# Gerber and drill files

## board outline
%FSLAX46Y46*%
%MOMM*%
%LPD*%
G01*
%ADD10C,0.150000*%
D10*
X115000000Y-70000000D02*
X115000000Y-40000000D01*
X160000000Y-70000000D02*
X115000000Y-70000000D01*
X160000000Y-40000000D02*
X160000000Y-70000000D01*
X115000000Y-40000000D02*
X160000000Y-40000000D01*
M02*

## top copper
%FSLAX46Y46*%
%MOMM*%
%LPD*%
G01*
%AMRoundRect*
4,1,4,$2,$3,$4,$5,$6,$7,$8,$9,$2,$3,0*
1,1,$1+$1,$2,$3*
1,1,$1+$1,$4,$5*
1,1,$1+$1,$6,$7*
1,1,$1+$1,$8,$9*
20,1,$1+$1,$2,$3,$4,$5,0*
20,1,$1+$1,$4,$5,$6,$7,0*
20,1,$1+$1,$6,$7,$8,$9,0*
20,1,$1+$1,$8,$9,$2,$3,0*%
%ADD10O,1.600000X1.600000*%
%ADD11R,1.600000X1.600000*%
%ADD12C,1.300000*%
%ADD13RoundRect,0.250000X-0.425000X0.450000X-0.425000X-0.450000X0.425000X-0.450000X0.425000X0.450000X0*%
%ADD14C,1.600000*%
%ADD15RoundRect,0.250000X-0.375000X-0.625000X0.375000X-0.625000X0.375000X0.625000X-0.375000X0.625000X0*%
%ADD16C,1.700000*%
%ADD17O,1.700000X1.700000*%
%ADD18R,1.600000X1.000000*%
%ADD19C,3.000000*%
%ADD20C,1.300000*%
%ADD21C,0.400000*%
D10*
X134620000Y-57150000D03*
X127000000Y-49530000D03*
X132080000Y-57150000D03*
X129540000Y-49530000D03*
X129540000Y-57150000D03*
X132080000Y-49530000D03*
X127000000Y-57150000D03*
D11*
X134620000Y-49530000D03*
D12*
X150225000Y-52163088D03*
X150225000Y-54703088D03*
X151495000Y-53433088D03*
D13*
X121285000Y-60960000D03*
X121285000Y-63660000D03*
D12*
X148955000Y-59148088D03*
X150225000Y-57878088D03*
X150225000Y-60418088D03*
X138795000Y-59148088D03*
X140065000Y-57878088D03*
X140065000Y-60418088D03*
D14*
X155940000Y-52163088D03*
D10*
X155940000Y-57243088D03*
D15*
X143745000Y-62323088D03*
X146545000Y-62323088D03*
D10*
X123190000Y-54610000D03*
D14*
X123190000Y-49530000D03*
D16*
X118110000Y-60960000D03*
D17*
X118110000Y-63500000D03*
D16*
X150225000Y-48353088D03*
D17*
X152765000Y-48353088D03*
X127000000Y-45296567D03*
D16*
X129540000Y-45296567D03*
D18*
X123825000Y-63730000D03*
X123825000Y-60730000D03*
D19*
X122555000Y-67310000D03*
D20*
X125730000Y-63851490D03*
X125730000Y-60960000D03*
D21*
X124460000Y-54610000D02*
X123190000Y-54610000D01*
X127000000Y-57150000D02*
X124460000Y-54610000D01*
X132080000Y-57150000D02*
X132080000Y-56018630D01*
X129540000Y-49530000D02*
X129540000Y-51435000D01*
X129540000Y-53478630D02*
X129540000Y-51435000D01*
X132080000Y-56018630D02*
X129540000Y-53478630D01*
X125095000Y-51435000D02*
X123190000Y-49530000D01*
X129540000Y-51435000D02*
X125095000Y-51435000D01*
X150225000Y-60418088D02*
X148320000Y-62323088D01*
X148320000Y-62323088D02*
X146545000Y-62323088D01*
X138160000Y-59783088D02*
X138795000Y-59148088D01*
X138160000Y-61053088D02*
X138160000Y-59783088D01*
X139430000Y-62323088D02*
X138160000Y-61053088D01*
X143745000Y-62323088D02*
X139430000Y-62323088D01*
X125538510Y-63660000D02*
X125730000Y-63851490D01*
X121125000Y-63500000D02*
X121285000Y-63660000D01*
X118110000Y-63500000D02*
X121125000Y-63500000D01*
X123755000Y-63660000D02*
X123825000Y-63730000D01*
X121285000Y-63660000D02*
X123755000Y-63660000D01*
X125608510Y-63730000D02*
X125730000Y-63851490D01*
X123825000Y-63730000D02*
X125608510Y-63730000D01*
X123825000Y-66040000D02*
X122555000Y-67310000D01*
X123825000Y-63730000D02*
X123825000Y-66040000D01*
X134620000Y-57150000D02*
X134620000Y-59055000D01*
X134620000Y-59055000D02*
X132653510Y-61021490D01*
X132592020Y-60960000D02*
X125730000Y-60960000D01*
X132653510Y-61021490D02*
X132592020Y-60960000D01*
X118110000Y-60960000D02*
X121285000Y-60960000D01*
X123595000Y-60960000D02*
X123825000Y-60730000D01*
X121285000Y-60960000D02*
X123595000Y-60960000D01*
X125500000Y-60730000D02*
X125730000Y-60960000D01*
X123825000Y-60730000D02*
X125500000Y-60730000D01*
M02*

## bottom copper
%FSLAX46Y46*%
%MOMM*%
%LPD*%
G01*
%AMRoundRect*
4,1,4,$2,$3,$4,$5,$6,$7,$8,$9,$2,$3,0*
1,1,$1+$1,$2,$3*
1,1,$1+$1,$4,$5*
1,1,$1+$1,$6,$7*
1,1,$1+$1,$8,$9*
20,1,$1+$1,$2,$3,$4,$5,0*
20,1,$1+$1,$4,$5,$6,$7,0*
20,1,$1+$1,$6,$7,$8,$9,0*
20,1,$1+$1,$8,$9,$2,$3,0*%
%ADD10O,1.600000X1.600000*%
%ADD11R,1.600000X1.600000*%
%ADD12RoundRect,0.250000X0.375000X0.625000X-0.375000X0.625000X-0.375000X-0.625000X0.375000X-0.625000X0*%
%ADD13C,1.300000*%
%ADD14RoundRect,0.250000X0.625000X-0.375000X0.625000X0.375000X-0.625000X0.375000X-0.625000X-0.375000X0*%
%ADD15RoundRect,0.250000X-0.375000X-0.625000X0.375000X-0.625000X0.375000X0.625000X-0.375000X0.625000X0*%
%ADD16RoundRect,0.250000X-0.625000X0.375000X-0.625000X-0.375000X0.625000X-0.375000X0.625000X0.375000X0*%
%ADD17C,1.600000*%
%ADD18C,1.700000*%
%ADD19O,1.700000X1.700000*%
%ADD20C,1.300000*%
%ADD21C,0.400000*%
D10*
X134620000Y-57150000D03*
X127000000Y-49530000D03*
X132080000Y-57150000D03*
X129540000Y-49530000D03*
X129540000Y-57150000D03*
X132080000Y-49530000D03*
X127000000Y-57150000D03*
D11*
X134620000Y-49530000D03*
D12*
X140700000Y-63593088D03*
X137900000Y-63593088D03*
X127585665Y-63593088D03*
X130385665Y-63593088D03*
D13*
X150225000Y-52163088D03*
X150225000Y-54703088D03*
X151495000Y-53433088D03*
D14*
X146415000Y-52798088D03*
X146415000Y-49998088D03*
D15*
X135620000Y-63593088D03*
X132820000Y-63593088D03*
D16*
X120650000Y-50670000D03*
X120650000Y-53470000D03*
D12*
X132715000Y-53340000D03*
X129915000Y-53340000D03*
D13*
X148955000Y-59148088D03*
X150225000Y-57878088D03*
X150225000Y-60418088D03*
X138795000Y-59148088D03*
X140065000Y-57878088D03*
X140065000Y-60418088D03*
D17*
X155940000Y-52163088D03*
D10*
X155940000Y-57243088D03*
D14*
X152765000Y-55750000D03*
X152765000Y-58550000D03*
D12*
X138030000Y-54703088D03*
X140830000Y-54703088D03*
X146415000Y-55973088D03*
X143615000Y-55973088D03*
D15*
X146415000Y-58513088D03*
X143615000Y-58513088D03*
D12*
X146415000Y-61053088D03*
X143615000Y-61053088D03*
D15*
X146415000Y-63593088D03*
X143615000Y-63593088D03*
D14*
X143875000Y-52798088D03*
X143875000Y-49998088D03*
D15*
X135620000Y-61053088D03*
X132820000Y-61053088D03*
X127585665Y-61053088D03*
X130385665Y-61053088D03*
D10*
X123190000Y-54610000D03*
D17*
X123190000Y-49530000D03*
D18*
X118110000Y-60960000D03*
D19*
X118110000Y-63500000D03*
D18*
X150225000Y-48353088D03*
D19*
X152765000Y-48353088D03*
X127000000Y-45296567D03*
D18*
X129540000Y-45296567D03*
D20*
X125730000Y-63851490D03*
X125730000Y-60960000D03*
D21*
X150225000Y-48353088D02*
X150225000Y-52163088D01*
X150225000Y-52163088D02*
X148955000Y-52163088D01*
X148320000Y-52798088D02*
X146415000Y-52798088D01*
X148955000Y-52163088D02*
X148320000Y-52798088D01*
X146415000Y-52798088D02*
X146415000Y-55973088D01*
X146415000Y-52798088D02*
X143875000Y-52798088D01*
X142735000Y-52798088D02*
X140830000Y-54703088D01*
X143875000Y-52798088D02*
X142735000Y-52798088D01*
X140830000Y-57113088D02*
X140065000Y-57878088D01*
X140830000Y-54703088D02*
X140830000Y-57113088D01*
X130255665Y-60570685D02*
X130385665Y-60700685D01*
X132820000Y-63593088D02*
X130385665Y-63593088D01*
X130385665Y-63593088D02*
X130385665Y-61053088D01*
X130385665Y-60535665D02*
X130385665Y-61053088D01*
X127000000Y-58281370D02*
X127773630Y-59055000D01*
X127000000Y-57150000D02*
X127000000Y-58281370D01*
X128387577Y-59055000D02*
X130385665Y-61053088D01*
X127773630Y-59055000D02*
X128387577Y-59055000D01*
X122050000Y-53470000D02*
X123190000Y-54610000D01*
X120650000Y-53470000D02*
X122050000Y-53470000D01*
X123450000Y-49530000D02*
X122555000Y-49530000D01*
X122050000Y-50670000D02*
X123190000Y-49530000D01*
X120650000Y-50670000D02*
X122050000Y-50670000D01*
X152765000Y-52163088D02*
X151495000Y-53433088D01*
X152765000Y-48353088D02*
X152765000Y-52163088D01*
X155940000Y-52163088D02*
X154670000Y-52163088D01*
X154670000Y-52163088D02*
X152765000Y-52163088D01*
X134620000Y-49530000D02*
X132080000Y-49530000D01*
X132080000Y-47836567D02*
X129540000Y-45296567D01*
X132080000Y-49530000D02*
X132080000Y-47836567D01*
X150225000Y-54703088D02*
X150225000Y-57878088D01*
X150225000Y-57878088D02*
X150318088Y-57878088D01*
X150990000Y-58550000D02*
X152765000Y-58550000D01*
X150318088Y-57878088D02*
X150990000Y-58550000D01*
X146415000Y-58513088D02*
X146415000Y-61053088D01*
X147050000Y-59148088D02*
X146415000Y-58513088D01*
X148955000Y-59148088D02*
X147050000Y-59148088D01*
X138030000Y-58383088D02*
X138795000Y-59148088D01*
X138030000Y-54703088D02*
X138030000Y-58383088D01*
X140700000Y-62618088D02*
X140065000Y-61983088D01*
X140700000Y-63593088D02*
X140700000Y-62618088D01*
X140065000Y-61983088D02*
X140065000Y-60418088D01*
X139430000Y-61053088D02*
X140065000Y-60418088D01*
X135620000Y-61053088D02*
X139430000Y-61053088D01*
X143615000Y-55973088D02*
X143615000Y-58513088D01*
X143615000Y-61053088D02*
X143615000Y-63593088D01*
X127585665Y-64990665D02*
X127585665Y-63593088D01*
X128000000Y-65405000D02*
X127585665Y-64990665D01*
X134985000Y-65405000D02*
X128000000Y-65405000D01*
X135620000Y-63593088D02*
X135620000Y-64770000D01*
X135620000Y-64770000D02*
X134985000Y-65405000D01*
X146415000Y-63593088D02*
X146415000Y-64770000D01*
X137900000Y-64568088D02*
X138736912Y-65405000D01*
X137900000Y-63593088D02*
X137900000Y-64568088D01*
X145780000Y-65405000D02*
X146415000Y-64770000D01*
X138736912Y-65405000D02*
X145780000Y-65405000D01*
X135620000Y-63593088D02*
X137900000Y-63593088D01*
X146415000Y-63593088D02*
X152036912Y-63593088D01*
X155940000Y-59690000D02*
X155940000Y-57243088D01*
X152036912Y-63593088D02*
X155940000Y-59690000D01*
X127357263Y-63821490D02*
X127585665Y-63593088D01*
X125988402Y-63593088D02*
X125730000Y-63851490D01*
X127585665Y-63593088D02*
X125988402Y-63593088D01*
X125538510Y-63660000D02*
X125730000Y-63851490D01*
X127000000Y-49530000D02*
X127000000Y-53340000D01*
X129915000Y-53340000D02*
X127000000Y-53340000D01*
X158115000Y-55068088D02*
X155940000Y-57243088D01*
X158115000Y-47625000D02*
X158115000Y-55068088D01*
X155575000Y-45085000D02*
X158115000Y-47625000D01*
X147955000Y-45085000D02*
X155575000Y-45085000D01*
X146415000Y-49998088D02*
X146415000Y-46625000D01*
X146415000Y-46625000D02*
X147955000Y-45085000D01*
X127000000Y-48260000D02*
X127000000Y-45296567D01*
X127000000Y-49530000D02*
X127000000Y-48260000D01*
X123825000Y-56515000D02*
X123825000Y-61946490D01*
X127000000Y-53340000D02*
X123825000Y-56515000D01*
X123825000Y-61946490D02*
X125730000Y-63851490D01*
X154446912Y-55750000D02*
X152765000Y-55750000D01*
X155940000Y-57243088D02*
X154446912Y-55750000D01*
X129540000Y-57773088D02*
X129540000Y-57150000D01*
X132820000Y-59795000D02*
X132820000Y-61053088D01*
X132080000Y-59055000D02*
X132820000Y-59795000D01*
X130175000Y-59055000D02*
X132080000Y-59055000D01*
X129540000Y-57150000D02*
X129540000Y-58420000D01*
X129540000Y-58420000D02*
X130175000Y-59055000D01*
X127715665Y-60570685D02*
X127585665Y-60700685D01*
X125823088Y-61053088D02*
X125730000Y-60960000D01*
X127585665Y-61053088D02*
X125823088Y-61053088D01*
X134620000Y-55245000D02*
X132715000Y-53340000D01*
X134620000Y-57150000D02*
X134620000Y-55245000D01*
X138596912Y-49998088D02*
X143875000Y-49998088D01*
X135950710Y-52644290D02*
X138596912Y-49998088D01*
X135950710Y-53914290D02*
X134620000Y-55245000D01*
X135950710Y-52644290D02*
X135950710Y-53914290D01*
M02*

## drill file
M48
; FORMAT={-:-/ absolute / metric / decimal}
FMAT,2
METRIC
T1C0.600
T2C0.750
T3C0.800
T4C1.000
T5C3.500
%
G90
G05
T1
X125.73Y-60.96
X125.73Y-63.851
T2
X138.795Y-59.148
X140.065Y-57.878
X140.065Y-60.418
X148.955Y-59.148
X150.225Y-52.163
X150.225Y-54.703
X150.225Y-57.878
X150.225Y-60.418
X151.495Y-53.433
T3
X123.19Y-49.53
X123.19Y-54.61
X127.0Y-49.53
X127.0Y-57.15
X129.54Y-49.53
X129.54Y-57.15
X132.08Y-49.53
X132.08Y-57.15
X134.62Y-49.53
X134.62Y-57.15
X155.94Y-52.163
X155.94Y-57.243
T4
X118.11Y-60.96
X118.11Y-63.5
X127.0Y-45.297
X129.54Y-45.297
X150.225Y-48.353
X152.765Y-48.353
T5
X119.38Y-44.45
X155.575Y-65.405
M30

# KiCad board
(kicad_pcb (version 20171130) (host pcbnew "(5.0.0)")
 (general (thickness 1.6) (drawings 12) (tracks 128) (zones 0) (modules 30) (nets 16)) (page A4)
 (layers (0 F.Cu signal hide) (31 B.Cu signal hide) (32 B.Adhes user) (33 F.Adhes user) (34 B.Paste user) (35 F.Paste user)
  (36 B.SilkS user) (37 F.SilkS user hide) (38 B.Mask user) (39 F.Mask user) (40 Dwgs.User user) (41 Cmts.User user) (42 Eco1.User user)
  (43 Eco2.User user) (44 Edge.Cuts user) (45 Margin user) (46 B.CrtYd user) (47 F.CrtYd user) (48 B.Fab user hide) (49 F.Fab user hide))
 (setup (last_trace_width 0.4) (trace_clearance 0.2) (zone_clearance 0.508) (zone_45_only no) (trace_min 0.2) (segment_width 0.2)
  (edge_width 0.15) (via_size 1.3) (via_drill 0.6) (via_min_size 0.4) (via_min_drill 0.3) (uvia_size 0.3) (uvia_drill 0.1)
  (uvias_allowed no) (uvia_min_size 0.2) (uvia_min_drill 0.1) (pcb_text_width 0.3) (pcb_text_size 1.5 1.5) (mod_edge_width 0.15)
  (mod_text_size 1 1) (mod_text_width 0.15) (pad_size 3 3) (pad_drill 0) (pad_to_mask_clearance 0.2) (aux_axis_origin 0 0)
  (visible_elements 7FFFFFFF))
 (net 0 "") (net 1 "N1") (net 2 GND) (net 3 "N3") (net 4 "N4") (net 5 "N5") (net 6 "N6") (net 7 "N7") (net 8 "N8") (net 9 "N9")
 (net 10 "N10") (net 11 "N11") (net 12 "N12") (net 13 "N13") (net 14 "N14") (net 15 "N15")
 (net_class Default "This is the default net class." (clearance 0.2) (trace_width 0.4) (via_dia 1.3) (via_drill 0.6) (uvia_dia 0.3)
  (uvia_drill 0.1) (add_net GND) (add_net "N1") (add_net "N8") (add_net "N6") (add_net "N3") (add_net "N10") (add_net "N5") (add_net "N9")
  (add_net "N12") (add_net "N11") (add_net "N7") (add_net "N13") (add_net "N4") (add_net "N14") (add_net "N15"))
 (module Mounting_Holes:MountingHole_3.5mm (layer F.Cu) (at 119.38 44.45)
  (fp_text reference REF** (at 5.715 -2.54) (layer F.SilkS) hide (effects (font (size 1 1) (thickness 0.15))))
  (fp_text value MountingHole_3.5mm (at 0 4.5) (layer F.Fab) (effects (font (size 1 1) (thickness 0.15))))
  (pad 1 np_thru_hole circle (at 0 0) (size 3.5 3.5) (drill 3.5) (layers *.Cu *.Mask)))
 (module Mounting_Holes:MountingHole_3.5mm (layer F.Cu) (at 155.575 65.405)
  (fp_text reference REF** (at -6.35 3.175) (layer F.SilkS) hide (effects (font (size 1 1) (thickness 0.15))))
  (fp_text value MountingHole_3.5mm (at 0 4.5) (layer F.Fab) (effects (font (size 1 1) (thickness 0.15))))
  (pad 1 np_thru_hole circle (at 0 0) (size 3.5 3.5) (drill 3.5) (layers *.Cu *.Mask)))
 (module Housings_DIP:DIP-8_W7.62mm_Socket (layer F.Cu) (at 134.62 49.53 270)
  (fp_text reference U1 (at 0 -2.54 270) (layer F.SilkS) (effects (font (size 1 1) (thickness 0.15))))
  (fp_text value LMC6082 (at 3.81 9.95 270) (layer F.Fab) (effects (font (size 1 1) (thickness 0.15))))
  (pad 8 thru_hole oval (at 7.62 0 270) (size 1.6 1.6) (drill 0.8) (layers *.Cu *.Mask) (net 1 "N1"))
  (pad 4 thru_hole oval (at 0 7.62 270) (size 1.6 1.6) (drill 0.8) (layers *.Cu *.Mask) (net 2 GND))
  (pad 7 thru_hole oval (at 7.62 2.54 270) (size 1.6 1.6) (drill 0.8) (layers *.Cu *.Mask) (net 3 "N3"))
  (pad 3 thru_hole oval (at 0 5.08 270) (size 1.6 1.6) (drill 0.8) (layers *.Cu *.Mask) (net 3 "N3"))
  (pad 6 thru_hole oval (at 7.62 5.08 270) (size 1.6 1.6) (drill 0.8) (layers *.Cu *.Mask) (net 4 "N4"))
  (pad 2 thru_hole oval (at 0 2.54 270) (size 1.6 1.6) (drill 0.8) (layers *.Cu *.Mask) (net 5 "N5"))
  (pad 5 thru_hole oval (at 7.62 7.62 270) (size 1.6 1.6) (drill 0.8) (layers *.Cu *.Mask) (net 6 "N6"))
  (pad 1 thru_hole rect (at 0 0 270) (size 1.6 1.6) (drill 0.8) (layers *.Cu *.Mask) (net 5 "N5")))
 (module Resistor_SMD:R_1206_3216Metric (layer B.Cu) (at 139.3 63.593088 180)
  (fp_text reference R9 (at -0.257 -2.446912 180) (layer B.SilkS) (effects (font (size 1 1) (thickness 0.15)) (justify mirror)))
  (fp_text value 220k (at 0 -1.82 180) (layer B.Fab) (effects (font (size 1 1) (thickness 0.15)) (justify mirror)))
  (pad 1 smd roundrect (at -1.4 0 180) (size 1.25 1.75) (layers B.Cu B.Paste B.Mask) (roundrect_rratio 0.2) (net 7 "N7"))
  (pad 2 smd roundrect (at 1.4 0 180) (size 1.25 1.75) (layers B.Cu B.Paste B.Mask) (roundrect_rratio 0.2) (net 2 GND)))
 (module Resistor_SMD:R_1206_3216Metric (layer B.Cu) (at 128.985665 63.593088 180)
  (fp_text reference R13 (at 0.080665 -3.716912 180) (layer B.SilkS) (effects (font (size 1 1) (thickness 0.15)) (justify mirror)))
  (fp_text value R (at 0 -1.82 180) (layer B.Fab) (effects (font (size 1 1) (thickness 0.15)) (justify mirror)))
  (pad 2 smd roundrect (at 1.4 0 180) (size 1.25 1.75) (layers B.Cu B.Paste B.Mask) (roundrect_rratio 0.2) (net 2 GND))
  (pad 1 smd roundrect (at -1.4 0 180) (size 1.25 1.75) (layers B.Cu B.Paste B.Mask) (roundrect_rratio 0.2) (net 6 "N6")))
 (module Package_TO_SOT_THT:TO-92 (layer F.Cu) (at 150.225 52.163088 270)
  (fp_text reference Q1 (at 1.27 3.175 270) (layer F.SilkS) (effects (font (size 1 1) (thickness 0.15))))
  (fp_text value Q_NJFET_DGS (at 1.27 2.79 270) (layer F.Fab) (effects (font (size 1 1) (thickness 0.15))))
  (pad 1 thru_hole circle (at 0 0) (size 1.3 1.3) (drill 0.75) (layers *.Cu *.Mask) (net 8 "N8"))
  (pad 3 thru_hole circle (at 2.54 0) (size 1.3 1.3) (drill 0.75) (layers *.Cu *.Mask) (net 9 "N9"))
  (pad 2 thru_hole circle (at 1.27 -1.27) (size 1.3 1.3) (drill 0.75) (layers *.Cu *.Mask) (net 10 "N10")))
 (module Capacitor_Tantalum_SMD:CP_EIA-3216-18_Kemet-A (layer F.Cu) (at 121.285 62.31 270)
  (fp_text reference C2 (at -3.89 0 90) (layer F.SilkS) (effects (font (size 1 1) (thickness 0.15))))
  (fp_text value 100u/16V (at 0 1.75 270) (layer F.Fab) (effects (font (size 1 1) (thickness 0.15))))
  (pad 1 smd roundrect (at -1.35 0 270) (size 1.4 1.35) (layers F.Cu F.Paste F.Mask) (roundrect_rratio 0.185185) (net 1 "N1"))
  (pad 2 smd roundrect (at 1.35 0 270) (size 1.4 1.35) (layers F.Cu F.Paste F.Mask) (roundrect_rratio 0.185185) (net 2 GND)))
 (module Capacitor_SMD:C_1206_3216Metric (layer B.Cu) (at 146.415 51.398088 90)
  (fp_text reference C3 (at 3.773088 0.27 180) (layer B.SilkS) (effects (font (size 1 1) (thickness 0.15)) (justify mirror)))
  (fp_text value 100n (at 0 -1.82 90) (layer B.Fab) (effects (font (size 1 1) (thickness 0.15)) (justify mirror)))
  (pad 1 smd roundrect (at -1.4 0 90) (size 1.25 1.75) (layers B.Cu B.Paste B.Mask) (roundrect_rratio 0.2) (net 8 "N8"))
  (pad 2 smd roundrect (at 1.4 0 90) (size 1.25 1.75) (layers B.Cu B.Paste B.Mask) (roundrect_rratio 0.2) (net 2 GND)))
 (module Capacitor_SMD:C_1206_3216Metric (layer B.Cu) (at 134.22 63.593088)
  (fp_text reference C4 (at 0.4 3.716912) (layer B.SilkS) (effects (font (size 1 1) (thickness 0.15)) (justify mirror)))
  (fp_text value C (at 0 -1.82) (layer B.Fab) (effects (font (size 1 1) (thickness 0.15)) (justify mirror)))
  (pad 2 smd roundrect (at 1.4 0) (size 1.25 1.75) (layers B.Cu B.Paste B.Mask) (roundrect_rratio 0.2) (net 2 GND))
  (pad 1 smd roundrect (at -1.4 0) (size 1.25 1.75) (layers B.Cu B.Paste B.Mask) (roundrect_rratio 0.2) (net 6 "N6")))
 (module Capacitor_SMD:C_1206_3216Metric (layer B.Cu) (at 120.65 52.07 270)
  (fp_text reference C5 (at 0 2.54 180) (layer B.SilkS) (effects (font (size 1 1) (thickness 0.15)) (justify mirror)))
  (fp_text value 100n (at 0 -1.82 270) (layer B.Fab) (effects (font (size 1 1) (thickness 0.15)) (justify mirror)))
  (pad 1 smd roundrect (at -1.4 0 270) (size 1.25 1.75) (layers B.Cu B.Paste B.Mask) (roundrect_rratio 0.2) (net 3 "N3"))
  (pad 2 smd roundrect (at 1.4 0 270) (size 1.25 1.75) (layers B.Cu B.Paste B.Mask) (roundrect_rratio 0.2) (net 6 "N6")))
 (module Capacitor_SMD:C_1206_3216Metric (layer B.Cu) (at 131.315 53.34 180)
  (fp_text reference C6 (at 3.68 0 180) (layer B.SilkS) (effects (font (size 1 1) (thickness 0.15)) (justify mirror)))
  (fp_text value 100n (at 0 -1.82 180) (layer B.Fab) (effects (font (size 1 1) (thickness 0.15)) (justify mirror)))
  (pad 1 smd roundrect (at -1.4 0 180) (size 1.25 1.75) (layers B.Cu B.Paste B.Mask) (roundrect_rratio 0.2) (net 1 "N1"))
  (pad 2 smd roundrect (at 1.4 0 180) (size 1.25 1.75) (layers B.Cu B.Paste B.Mask) (roundrect_rratio 0.2) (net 2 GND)))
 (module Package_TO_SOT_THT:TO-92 (layer F.Cu) (at 150.225 60.418088 90)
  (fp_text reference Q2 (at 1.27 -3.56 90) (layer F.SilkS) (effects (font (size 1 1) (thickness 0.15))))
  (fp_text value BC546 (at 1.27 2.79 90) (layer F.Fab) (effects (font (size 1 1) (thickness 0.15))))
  (pad 2 thru_hole circle (at 1.27 -1.27 180) (size 1.3 1.3) (drill 0.75) (layers *.Cu *.Mask) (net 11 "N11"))
  (pad 3 thru_hole circle (at 2.54 0 180) (size 1.3 1.3) (drill 0.75) (layers *.Cu *.Mask) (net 9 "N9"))
  (pad 1 thru_hole circle (at 0 0 180) (size 1.3 1.3) (drill 0.75) (layers *.Cu *.Mask) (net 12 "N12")))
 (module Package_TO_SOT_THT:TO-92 (layer F.Cu) (at 140.065 60.418088 90)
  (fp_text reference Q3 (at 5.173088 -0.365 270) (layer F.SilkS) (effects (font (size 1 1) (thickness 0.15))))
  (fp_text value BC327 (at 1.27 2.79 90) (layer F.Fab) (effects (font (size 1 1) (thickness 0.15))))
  (pad 2 thru_hole circle (at 1.27 -1.27 180) (size 1.3 1.3) (drill 0.75) (layers *.Cu *.Mask) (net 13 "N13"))
  (pad 3 thru_hole circle (at 2.54 0 180) (size 1.3 1.3) (drill 0.75) (layers *.Cu *.Mask) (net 8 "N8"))
  (pad 1 thru_hole circle (at 0 0 180) (size 1.3 1.3) (drill 0.75) (layers *.Cu *.Mask) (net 7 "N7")))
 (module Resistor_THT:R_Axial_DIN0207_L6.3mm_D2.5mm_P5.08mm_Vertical (layer F.Cu) (at 155.94 52.163088 270)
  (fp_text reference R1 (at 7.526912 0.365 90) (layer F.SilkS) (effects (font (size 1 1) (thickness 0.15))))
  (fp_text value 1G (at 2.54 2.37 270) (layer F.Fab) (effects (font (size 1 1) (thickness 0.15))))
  (pad 1 thru_hole circle (at 0 0 270) (size 1.6 1.6) (drill 0.8) (layers *.Cu *.Mask) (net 10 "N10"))
  (pad 2 thru_hole oval (at 5.08 0 270) (size 1.6 1.6) (drill 0.8) (layers *.Cu *.Mask) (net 2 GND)))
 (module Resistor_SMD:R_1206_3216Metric (layer B.Cu) (at 152.765 57.15 90)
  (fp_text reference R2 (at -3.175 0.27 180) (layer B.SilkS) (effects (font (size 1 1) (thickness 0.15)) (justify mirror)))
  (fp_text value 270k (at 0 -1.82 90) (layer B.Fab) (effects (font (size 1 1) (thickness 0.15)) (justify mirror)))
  (pad 2 smd roundrect (at 1.4 0 90) (size 1.25 1.75) (layers B.Cu B.Paste B.Mask) (roundrect_rratio 0.2) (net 2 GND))
  (pad 1 smd roundrect (at -1.4 0 90) (size 1.25 1.75) (layers B.Cu B.Paste B.Mask) (roundrect_rratio 0.2) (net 9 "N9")))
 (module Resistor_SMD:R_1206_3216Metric (layer B.Cu) (at 139.43 54.703088 180)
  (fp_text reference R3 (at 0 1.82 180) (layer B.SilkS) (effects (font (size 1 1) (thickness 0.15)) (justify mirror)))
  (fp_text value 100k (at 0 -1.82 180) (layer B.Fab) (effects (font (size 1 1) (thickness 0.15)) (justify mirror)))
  (pad 2 smd roundrect (at 1.4 0 180) (size 1.25 1.75) (layers B.Cu B.Paste B.Mask) (roundrect_rratio 0.2) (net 13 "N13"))
  (pad 1 smd roundrect (at -1.4 0 180) (size 1.25 1.75) (layers B.Cu B.Paste B.Mask) (roundrect_rratio 0.2) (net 8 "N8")))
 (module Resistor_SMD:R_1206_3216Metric (layer F.Cu) (at 145.145 62.323088)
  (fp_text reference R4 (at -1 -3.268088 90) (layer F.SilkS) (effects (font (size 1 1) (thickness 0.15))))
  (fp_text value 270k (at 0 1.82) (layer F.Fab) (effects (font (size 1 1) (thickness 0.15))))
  (pad 1 smd roundrect (at -1.4 0) (size 1.25 1.75) (layers F.Cu F.Paste F.Mask) (roundrect_rratio 0.2) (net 13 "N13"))
  (pad 2 smd roundrect (at 1.4 0) (size 1.25 1.75) (layers F.Cu F.Paste F.Mask) (roundrect_rratio 0.2) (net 12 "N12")))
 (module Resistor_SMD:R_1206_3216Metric (layer B.Cu) (at 145.015 55.973088 180)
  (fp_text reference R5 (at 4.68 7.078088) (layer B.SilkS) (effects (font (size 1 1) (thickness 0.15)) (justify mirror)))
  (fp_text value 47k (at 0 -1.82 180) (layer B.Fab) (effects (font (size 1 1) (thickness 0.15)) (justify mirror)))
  (pad 1 smd roundrect (at -1.4 0 180) (size 1.25 1.75) (layers B.Cu B.Paste B.Mask) (roundrect_rratio 0.2) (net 8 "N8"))
  (pad 2 smd roundrect (at 1.4 0 180) (size 1.25 1.75) (layers B.Cu B.Paste B.Mask) (roundrect_rratio 0.2) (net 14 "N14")))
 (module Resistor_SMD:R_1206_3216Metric (layer B.Cu) (at 145.015 58.513088)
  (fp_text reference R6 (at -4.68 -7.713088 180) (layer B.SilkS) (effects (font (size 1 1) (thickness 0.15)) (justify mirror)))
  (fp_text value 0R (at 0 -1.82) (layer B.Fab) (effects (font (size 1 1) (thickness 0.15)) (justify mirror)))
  (pad 2 smd roundrect (at 1.4 0) (size 1.25 1.75) (layers B.Cu B.Paste B.Mask) (roundrect_rratio 0.2) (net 11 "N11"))
  (pad 1 smd roundrect (at -1.4 0) (size 1.25 1.75) (layers B.Cu B.Paste B.Mask) (roundrect_rratio 0.2) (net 14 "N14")))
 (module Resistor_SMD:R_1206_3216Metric (layer B.Cu) (at 145.015 61.053088 180)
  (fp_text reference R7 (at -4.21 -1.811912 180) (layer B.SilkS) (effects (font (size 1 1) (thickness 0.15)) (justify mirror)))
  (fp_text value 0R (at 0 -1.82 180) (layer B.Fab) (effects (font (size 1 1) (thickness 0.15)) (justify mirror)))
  (pad 1 smd roundrect (at -1.4 0 180) (size 1.25 1.75) (layers B.Cu B.Paste B.Mask) (roundrect_rratio 0.2) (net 11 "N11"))
  (pad 2 smd roundrect (at 1.4 0 180) (size 1.25 1.75) (layers B.Cu B.Paste B.Mask) (roundrect_rratio 0.2) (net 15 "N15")))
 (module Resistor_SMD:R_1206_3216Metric (layer B.Cu) (at 145.015 63.593088)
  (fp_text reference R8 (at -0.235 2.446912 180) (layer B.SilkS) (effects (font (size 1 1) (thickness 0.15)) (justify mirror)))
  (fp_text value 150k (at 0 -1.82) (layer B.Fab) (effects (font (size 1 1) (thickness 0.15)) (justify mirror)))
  (pad 2 smd roundrect (at 1.4 0) (size 1.25 1.75) (layers B.Cu B.Paste B.Mask) (roundrect_rratio 0.2) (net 2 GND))
  (pad 1 smd roundrect (at -1.4 0) (size 1.25 1.75) (layers B.Cu B.Paste B.Mask) (roundrect_rratio 0.2) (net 15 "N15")))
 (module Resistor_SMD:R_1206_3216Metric (layer B.Cu) (at 143.875 51.398088 90)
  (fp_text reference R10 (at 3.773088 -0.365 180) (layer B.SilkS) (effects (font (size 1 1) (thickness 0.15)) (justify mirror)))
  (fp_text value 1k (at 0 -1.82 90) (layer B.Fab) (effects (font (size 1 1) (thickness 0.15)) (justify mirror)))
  (pad 1 smd roundrect (at -1.4 0 90) (size 1.25 1.75) (layers B.Cu B.Paste B.Mask) (roundrect_rratio 0.2) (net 8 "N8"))
  (pad 2 smd roundrect (at 1.4 0 90) (size 1.25 1.75) (layers B.Cu B.Paste B.Mask) (roundrect_rratio 0.2) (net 1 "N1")))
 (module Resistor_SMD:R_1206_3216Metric (layer B.Cu) (at 134.22 61.053088)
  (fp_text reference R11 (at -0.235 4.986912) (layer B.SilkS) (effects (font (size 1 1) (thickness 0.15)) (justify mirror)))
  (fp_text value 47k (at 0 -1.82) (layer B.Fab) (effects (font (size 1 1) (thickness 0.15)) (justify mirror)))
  (pad 2 smd roundrect (at 1.4 0) (size 1.25 1.75) (layers B.Cu B.Paste B.Mask) (roundrect_rratio 0.2) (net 7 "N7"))
  (pad 1 smd roundrect (at -1.4 0) (size 1.25 1.75) (layers B.Cu B.Paste B.Mask) (roundrect_rratio 0.2) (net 4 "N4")))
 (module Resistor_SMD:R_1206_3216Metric (layer B.Cu) (at 128.985665 61.053088)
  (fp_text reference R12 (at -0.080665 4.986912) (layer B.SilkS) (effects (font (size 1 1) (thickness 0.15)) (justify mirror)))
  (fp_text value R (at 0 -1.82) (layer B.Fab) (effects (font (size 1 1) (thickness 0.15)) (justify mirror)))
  (pad 1 smd roundrect (at -1.4 0) (size 1.25 1.75) (layers B.Cu B.Paste B.Mask) (roundrect_rratio 0.2) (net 1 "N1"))
  (pad 2 smd roundrect (at 1.4 0) (size 1.25 1.75) (layers B.Cu B.Paste B.Mask) (roundrect_rratio 0.2) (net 6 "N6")))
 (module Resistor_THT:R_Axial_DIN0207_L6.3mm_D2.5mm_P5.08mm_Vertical (layer F.Cu) (at 123.19 49.53 270)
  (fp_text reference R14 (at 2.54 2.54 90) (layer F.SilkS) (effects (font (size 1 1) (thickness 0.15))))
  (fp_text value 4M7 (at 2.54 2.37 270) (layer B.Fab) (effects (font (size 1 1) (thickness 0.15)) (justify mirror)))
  (pad 2 thru_hole oval (at 5.08 0 270) (size 1.6 1.6) (drill 0.8) (layers *.Cu *.Mask) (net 6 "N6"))
  (pad 1 thru_hole circle (at 0 0 270) (size 1.6 1.6) (drill 0.8) (layers *.Cu *.Mask) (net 3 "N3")))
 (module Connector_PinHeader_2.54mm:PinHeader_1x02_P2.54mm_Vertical (layer F.Cu) (at 118.11 60.96)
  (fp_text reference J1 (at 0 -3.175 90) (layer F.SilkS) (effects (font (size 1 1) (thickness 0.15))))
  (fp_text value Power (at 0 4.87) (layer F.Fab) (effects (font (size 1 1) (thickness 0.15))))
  (pad 1 thru_hole circle (at 0 0) (size 1.7 1.7) (drill 1) (layers *.Cu *.Mask) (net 1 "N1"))
  (pad 2 thru_hole oval (at 0 2.54) (size 1.7 1.7) (drill 1) (layers *.Cu *.Mask) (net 2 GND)))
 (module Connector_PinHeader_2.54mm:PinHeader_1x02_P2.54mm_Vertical (layer F.Cu) (at 150.225 48.353088 90)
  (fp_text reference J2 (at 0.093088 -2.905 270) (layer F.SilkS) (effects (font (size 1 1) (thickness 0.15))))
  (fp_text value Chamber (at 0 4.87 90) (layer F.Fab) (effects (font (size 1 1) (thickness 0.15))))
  (pad 1 thru_hole circle (at 0 0 90) (size 1.7 1.7) (drill 1) (layers *.Cu *.Mask) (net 8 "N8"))
  (pad 2 thru_hole oval (at 0 2.54 90) (size 1.7 1.7) (drill 1) (layers *.Cu *.Mask) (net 10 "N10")))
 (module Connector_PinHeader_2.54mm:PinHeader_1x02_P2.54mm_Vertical (layer F.Cu) (at 129.54 45.296567 270)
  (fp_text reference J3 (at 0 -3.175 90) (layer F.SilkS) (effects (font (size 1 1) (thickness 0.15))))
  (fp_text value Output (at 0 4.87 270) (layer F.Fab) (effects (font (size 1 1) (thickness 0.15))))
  (pad 2 thru_hole oval (at 0 2.54 270) (size 1.7 1.7) (drill 1) (layers *.Cu *.Mask) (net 2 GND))
  (pad 1 thru_hole circle (at 0 0 270) (size 1.7 1.7) (drill 1) (layers *.Cu *.Mask) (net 5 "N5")))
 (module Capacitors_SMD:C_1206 (layer F.Cu) (at 123.825 62.23 270)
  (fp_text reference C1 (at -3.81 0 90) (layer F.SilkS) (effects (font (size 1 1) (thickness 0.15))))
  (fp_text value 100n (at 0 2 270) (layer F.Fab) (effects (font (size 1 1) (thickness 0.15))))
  (pad 2 smd rect (at 1.5 0 270) (size 1 1.6) (layers F.Cu F.Paste F.Mask) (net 2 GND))
  (pad 1 smd rect (at -1.5 0 270) (size 1 1.6) (layers F.Cu F.Paste F.Mask) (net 1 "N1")))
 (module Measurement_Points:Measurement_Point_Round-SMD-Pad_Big (layer F.Cu) (at 122.555 67.31)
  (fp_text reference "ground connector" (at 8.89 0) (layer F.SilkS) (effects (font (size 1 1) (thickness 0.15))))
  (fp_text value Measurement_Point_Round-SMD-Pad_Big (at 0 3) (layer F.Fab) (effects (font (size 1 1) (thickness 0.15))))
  (pad 1 smd circle (at 0 0) (size 3 3) (layers F.Cu F.Mask) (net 2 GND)))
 (gr_line (start 115 70) (end 115 40) (layer Edge.Cuts) (width 0.15))
 (gr_line (start 160 70) (end 115 70) (layer Edge.Cuts) (width 0.15))
 (gr_line (start 160 40) (end 160 70) (layer Edge.Cuts) (width 0.15))
 (gr_line (start 115 40) (end 160 40) (layer Edge.Cuts) (width 0.15))
 (segment (start 150.225 48.353088) (end 150.225 52.163088) (width 0.4) (layer B.Cu) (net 8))
 (segment (start 150.225 52.163088) (end 148.955 52.163088) (width 0.4) (layer B.Cu) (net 8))
 (segment (start 148.32 52.798088) (end 146.415 52.798088) (width 0.4) (layer B.Cu) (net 8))
 (segment (start 148.955 52.163088) (end 148.32 52.798088) (width 0.4) (layer B.Cu) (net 8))
 (segment (start 146.415 52.798088) (end 146.415 55.973088) (width 0.4) (layer B.Cu) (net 8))
 (segment (start 146.415 52.798088) (end 143.875 52.798088) (width 0.4) (layer B.Cu) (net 8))
 (segment (start 142.735 52.798088) (end 140.83 54.703088) (width 0.4) (layer B.Cu) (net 8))
 (segment (start 143.875 52.798088) (end 142.735 52.798088) (width 0.4) (layer B.Cu) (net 8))
 (segment (start 140.83 57.113088) (end 140.065 57.878088) (width 0.4) (layer B.Cu) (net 8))
 (segment (start 140.83 54.703088) (end 140.83 57.113088) (width 0.4) (layer B.Cu) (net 8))
 (segment (start 130.255665 60.570685) (end 130.385665 60.700685) (width 0.4) (layer B.Cu) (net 6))
 (segment (start 132.82 63.593088) (end 130.385665 63.593088) (width 0.4) (layer B.Cu) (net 6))
 (segment (start 130.385665 63.593088) (end 130.385665 61.053088) (width 0.4) (layer B.Cu) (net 6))
 (segment (start 130.385665 60.535665) (end 130.385665 61.053088) (width 0.4) (layer B.Cu) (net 6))
 (segment (start 127 58.28137) (end 127.77363 59.055) (width 0.4) (layer B.Cu) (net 6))
 (segment (start 127 57.15) (end 127 58.28137) (width 0.4) (layer B.Cu) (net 6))
 (segment (start 128.387577 59.055) (end 130.385665 61.053088) (width 0.4) (layer B.Cu) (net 6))
 (segment (start 127.77363 59.055) (end 128.387577 59.055) (width 0.4) (layer B.Cu) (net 6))
 (segment (start 122.05 53.47) (end 123.19 54.61) (width 0.4) (layer B.Cu) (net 6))
 (segment (start 120.65 53.47) (end 122.05 53.47) (width 0.4) (layer B.Cu) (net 6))
 (segment (start 124.46 54.61) (end 123.19 54.61) (width 0.4) (layer F.Cu) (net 6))
 (segment (start 127 57.15) (end 124.46 54.61) (width 0.4) (layer F.Cu) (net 6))
 (segment (start 123.45 49.53) (end 122.555 49.53) (width 0.4) (layer B.Cu) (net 3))
 (segment (start 122.05 50.67) (end 123.19 49.53) (width 0.4) (layer B.Cu) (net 3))
 (segment (start 120.65 50.67) (end 122.05 50.67) (width 0.4) (layer B.Cu) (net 3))
 (segment (start 132.08 57.15) (end 132.08 56.01863) (width 0.4) (layer F.Cu) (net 3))
 (segment (start 129.54 49.53) (end 129.54 51.435) (width 0.4) (layer F.Cu) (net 3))
 (segment (start 129.54 53.47863) (end 129.54 51.435) (width 0.4) (layer F.Cu) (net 3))
 (segment (start 132.08 56.01863) (end 129.54 53.47863) (width 0.4) (layer F.Cu) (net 3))
 (segment (start 125.095 51.435) (end 123.19 49.53) (width 0.4) (layer F.Cu) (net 3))
 (segment (start 129.54 51.435) (end 125.095 51.435) (width 0.4) (layer F.Cu) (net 3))
 (segment (start 152.765 52.163088) (end 151.495 53.433088) (width 0.4) (layer B.Cu) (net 10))
 (segment (start 152.765 48.353088) (end 152.765 52.163088) (width 0.4) (layer B.Cu) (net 10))
 (segment (start 155.94 52.163088) (end 154.67 52.163088) (width 0.4) (layer B.Cu) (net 10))
 (segment (start 154.67 52.163088) (end 152.765 52.163088) (width 0.4) (layer B.Cu) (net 10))
 (segment (start 134.62 49.53) (end 132.08 49.53) (width 0.4) (layer B.Cu) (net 5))
 (segment (start 132.08 47.836567) (end 129.54 45.296567) (width 0.4) (layer B.Cu) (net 5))
 (segment (start 132.08 49.53) (end 132.08 47.836567) (width 0.4) (layer B.Cu) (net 5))
 (segment (start 150.225 54.703088) (end 150.225 57.878088) (width 0.4) (layer B.Cu) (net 9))
 (segment (start 150.225 57.878088) (end 150.318088 57.878088) (width 0.4) (layer B.Cu) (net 9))
 (segment (start 150.99 58.55) (end 152.765 58.55) (width 0.4) (layer B.Cu) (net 9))
 (segment (start 150.318088 57.878088) (end 150.99 58.55) (width 0.4) (layer B.Cu) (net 9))
 (segment (start 146.415 58.513088) (end 146.415 61.053088) (width 0.4) (layer B.Cu) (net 11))
 (segment (start 147.05 59.148088) (end 146.415 58.513088) (width 0.4) (layer B.Cu) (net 11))
 (segment (start 148.955 59.148088) (end 147.05 59.148088) (width 0.4) (layer B.Cu) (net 11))
 (segment (start 150.225 60.418088) (end 148.32 62.323088) (width 0.4) (layer F.Cu) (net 12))
 (segment (start 148.32 62.323088) (end 146.545 62.323088) (width 0.4) (layer F.Cu) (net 12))
 (segment (start 138.03 58.383088) (end 138.795 59.148088) (width 0.4) (layer B.Cu) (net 13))
 (segment (start 138.03 54.703088) (end 138.03 58.383088) (width 0.4) (layer B.Cu) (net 13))
 (segment (start 138.16 59.783088) (end 138.795 59.148088) (width 0.4) (layer F.Cu) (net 13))
 (segment (start 138.16 61.053088) (end 138.16 59.783088) (width 0.4) (layer F.Cu) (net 13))
 (segment (start 139.43 62.323088) (end 138.16 61.053088) (width 0.4) (layer F.Cu) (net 13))
 (segment (start 143.745 62.323088) (end 139.43 62.323088) (width 0.4) (layer F.Cu) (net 13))
 (segment (start 140.7 62.618088) (end 140.065 61.983088) (width 0.4) (layer B.Cu) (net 7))
 (segment (start 140.7 63.593088) (end 140.7 62.618088) (width 0.4) (layer B.Cu) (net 7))
 (segment (start 140.065 61.983088) (end 140.065 60.418088) (width 0.4) (layer B.Cu) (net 7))
 (segment (start 139.43 61.053088) (end 140.065 60.418088) (width 0.4) (layer B.Cu) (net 7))
 (segment (start 135.62 61.053088) (end 139.43 61.053088) (width 0.4) (layer B.Cu) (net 7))
 (segment (start 143.615 55.973088) (end 143.615 58.513088) (width 0.4) (layer B.Cu) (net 14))
 (segment (start 143.615 61.053088) (end 143.615 63.593088) (width 0.4) (layer B.Cu) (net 15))
 (segment (start 127.585665 64.990665) (end 127.585665 63.593088) (width 0.4) (layer B.Cu) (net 2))
 (segment (start 128 65.405) (end 127.585665 64.990665) (width 0.4) (layer B.Cu) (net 2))
 (segment (start 134.985 65.405) (end 128 65.405) (width 0.4) (layer B.Cu) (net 2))
 (segment (start 135.62 63.593088) (end 135.62 64.77) (width 0.4) (layer B.Cu) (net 2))
 (segment (start 135.62 64.77) (end 134.985 65.405) (width 0.4) (layer B.Cu) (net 2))
 (segment (start 146.415 63.593088) (end 146.415 64.77) (width 0.4) (layer B.Cu) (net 2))
 (segment (start 137.9 64.568088) (end 138.736912 65.405) (width 0.4) (layer B.Cu) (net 2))
 (segment (start 137.9 63.593088) (end 137.9 64.568088) (width 0.4) (layer B.Cu) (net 2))
 (segment (start 145.78 65.405) (end 146.415 64.77) (width 0.4) (layer B.Cu) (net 2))
 (segment (start 138.736912 65.405) (end 145.78 65.405) (width 0.4) (layer B.Cu) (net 2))
 (segment (start 135.62 63.593088) (end 137.9 63.593088) (width 0.4) (layer B.Cu) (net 2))
 (segment (start 146.415 63.593088) (end 152.036912 63.593088) (width 0.4) (layer B.Cu) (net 2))
 (segment (start 155.94 59.69) (end 155.94 57.243088) (width 0.4) (layer B.Cu) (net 2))
 (segment (start 152.036912 63.593088) (end 155.94 59.69) (width 0.4) (layer B.Cu) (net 2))
 (segment (start 127.357263 63.82149) (end 127.585665 63.593088) (width 0.4) (layer B.Cu) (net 2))
 (via (at 125.73 63.85149) (size 1.3) (drill 0.6) (layers F.Cu B.Cu) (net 2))
 (segment (start 125.988402 63.593088) (end 125.73 63.85149) (width 0.4) (layer B.Cu) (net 2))
 (segment (start 127.585665 63.593088) (end 125.988402 63.593088) (width 0.4) (layer B.Cu) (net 2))
 (segment (start 125.53851 63.66) (end 125.73 63.85149) (width 0.4) (layer B.Cu) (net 2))
 (segment (start 127 49.53) (end 127 53.34) (width 0.4) (layer B.Cu) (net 2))
 (segment (start 129.915 53.34) (end 127 53.34) (width 0.4) (layer B.Cu) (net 2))
 (segment (start 125.53851 63.66) (end 125.73 63.85149) (width 0.4) (layer F.Cu) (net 2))
 (segment (start 121.125 63.5) (end 121.285 63.66) (width 0.4) (layer F.Cu) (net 2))
 (segment (start 118.11 63.5) (end 121.125 63.5) (width 0.4) (layer F.Cu) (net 2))
 (segment (start 123.755 63.66) (end 123.825 63.73) (width 0.4) (layer F.Cu) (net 2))
 (segment (start 121.285 63.66) (end 123.755 63.66) (width 0.4) (layer F.Cu) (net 2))
 (segment (start 125.60851 63.73) (end 125.73 63.85149) (width 0.4) (layer F.Cu) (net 2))
 (segment (start 123.825 63.73) (end 125.60851 63.73) (width 0.4) (layer F.Cu) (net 2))
 (segment (start 158.115 55.068088) (end 155.94 57.243088) (width 0.4) (layer B.Cu) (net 2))
 (segment (start 158.115 47.625) (end 158.115 55.068088) (width 0.4) (layer B.Cu) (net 2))
 (segment (start 155.575 45.085) (end 158.115 47.625) (width 0.4) (layer B.Cu) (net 2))
 (segment (start 147.955 45.085) (end 155.575 45.085) (width 0.4) (layer B.Cu) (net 2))
 (segment (start 146.415 49.998088) (end 146.415 46.625) (width 0.4) (layer B.Cu) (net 2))
 (segment (start 146.415 46.625) (end 147.955 45.085) (width 0.4) (layer B.Cu) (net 2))
 (segment (start 127 48.26) (end 127 45.296567) (width 0.4) (layer B.Cu) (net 2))
 (segment (start 127 49.53) (end 127 48.26) (width 0.4) (layer B.Cu) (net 2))
 (segment (start 123.825 56.515) (end 123.825 61.94649) (width 0.4) (layer B.Cu) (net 2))
 (segment (start 127 53.34) (end 123.825 56.515) (width 0.4) (layer B.Cu) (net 2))
 (segment (start 123.825 61.94649) (end 125.73 63.85149) (width 0.4) (layer B.Cu) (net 2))
 (segment (start 154.446912 55.75) (end 152.765 55.75) (width 0.4) (layer B.Cu) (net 2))
 (segment (start 155.94 57.243088) (end 154.446912 55.75) (width 0.4) (layer B.Cu) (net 2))
 (segment (start 123.825 66.04) (end 122.555 67.31) (width 0.4) (layer F.Cu) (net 2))
 (segment (start 123.825 63.73) (end 123.825 66.04) (width 0.4) (layer F.Cu) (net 2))
 (segment (start 129.54 57.773088) (end 129.54 57.15) (width 0.4) (layer B.Cu) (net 4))
 (segment (start 132.82 59.795) (end 132.82 61.053088) (width 0.4) (layer B.Cu) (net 4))
 (segment (start 132.08 59.055) (end 132.82 59.795) (width 0.4) (layer B.Cu) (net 4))
 (segment (start 130.175 59.055) (end 132.08 59.055) (width 0.4) (layer B.Cu) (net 4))
 (segment (start 129.54 57.15) (end 129.54 58.42) (width 0.4) (layer B.Cu) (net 4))
 (segment (start 129.54 58.42) (end 130.175 59.055) (width 0.4) (layer B.Cu) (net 4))
 (segment (start 127.715665 60.570685) (end 127.585665 60.700685) (width 0.4) (layer B.Cu) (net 1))
 (via (at 125.73 60.96) (size 1.3) (drill 0.6) (layers F.Cu B.Cu) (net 1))
 (segment (start 134.62 57.15) (end 134.62 59.055) (width 0.4) (layer F.Cu) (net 1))
 (segment (start 134.62 59.055) (end 132.65351 61.02149) (width 0.4) (layer F.Cu) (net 1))
 (segment (start 125.823088 61.053088) (end 125.73 60.96) (width 0.4) (layer B.Cu) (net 1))
 (segment (start 127.585665 61.053088) (end 125.823088 61.053088) (width 0.4) (layer B.Cu) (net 1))
 (segment (start 132.59202 60.96) (end 125.73 60.96) (width 0.4) (layer F.Cu) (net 1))
 (segment (start 132.65351 61.02149) (end 132.59202 60.96) (width 0.4) (layer F.Cu) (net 1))
 (segment (start 134.62 55.245) (end 132.715 53.34) (width 0.4) (layer B.Cu) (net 1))
 (segment (start 134.62 57.15) (end 134.62 55.245) (width 0.4) (layer B.Cu) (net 1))
 (segment (start 138.596912 49.998088) (end 143.875 49.998088) (width 0.4) (layer B.Cu) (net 1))
 (segment (start 135.95071 52.64429) (end 138.596912 49.998088) (width 0.4) (layer B.Cu) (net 1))
 (segment (start 118.11 60.96) (end 121.285 60.96) (width 0.4) (layer F.Cu) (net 1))
 (segment (start 123.595 60.96) (end 123.825 60.73) (width 0.4) (layer F.Cu) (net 1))
 (segment (start 121.285 60.96) (end 123.595 60.96) (width 0.4) (layer F.Cu) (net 1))
 (segment (start 125.5 60.73) (end 125.73 60.96) (width 0.4) (layer F.Cu) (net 1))
 (segment (start 123.825 60.73) (end 125.5 60.73) (width 0.4) (layer F.Cu) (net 1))
 (segment (start 135.95071 53.91429) (end 134.62 55.245) (width 0.4) (layer B.Cu) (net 1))
 (segment (start 135.95071 52.64429) (end 135.95071 53.91429) (width 0.4) (layer B.Cu) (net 1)))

